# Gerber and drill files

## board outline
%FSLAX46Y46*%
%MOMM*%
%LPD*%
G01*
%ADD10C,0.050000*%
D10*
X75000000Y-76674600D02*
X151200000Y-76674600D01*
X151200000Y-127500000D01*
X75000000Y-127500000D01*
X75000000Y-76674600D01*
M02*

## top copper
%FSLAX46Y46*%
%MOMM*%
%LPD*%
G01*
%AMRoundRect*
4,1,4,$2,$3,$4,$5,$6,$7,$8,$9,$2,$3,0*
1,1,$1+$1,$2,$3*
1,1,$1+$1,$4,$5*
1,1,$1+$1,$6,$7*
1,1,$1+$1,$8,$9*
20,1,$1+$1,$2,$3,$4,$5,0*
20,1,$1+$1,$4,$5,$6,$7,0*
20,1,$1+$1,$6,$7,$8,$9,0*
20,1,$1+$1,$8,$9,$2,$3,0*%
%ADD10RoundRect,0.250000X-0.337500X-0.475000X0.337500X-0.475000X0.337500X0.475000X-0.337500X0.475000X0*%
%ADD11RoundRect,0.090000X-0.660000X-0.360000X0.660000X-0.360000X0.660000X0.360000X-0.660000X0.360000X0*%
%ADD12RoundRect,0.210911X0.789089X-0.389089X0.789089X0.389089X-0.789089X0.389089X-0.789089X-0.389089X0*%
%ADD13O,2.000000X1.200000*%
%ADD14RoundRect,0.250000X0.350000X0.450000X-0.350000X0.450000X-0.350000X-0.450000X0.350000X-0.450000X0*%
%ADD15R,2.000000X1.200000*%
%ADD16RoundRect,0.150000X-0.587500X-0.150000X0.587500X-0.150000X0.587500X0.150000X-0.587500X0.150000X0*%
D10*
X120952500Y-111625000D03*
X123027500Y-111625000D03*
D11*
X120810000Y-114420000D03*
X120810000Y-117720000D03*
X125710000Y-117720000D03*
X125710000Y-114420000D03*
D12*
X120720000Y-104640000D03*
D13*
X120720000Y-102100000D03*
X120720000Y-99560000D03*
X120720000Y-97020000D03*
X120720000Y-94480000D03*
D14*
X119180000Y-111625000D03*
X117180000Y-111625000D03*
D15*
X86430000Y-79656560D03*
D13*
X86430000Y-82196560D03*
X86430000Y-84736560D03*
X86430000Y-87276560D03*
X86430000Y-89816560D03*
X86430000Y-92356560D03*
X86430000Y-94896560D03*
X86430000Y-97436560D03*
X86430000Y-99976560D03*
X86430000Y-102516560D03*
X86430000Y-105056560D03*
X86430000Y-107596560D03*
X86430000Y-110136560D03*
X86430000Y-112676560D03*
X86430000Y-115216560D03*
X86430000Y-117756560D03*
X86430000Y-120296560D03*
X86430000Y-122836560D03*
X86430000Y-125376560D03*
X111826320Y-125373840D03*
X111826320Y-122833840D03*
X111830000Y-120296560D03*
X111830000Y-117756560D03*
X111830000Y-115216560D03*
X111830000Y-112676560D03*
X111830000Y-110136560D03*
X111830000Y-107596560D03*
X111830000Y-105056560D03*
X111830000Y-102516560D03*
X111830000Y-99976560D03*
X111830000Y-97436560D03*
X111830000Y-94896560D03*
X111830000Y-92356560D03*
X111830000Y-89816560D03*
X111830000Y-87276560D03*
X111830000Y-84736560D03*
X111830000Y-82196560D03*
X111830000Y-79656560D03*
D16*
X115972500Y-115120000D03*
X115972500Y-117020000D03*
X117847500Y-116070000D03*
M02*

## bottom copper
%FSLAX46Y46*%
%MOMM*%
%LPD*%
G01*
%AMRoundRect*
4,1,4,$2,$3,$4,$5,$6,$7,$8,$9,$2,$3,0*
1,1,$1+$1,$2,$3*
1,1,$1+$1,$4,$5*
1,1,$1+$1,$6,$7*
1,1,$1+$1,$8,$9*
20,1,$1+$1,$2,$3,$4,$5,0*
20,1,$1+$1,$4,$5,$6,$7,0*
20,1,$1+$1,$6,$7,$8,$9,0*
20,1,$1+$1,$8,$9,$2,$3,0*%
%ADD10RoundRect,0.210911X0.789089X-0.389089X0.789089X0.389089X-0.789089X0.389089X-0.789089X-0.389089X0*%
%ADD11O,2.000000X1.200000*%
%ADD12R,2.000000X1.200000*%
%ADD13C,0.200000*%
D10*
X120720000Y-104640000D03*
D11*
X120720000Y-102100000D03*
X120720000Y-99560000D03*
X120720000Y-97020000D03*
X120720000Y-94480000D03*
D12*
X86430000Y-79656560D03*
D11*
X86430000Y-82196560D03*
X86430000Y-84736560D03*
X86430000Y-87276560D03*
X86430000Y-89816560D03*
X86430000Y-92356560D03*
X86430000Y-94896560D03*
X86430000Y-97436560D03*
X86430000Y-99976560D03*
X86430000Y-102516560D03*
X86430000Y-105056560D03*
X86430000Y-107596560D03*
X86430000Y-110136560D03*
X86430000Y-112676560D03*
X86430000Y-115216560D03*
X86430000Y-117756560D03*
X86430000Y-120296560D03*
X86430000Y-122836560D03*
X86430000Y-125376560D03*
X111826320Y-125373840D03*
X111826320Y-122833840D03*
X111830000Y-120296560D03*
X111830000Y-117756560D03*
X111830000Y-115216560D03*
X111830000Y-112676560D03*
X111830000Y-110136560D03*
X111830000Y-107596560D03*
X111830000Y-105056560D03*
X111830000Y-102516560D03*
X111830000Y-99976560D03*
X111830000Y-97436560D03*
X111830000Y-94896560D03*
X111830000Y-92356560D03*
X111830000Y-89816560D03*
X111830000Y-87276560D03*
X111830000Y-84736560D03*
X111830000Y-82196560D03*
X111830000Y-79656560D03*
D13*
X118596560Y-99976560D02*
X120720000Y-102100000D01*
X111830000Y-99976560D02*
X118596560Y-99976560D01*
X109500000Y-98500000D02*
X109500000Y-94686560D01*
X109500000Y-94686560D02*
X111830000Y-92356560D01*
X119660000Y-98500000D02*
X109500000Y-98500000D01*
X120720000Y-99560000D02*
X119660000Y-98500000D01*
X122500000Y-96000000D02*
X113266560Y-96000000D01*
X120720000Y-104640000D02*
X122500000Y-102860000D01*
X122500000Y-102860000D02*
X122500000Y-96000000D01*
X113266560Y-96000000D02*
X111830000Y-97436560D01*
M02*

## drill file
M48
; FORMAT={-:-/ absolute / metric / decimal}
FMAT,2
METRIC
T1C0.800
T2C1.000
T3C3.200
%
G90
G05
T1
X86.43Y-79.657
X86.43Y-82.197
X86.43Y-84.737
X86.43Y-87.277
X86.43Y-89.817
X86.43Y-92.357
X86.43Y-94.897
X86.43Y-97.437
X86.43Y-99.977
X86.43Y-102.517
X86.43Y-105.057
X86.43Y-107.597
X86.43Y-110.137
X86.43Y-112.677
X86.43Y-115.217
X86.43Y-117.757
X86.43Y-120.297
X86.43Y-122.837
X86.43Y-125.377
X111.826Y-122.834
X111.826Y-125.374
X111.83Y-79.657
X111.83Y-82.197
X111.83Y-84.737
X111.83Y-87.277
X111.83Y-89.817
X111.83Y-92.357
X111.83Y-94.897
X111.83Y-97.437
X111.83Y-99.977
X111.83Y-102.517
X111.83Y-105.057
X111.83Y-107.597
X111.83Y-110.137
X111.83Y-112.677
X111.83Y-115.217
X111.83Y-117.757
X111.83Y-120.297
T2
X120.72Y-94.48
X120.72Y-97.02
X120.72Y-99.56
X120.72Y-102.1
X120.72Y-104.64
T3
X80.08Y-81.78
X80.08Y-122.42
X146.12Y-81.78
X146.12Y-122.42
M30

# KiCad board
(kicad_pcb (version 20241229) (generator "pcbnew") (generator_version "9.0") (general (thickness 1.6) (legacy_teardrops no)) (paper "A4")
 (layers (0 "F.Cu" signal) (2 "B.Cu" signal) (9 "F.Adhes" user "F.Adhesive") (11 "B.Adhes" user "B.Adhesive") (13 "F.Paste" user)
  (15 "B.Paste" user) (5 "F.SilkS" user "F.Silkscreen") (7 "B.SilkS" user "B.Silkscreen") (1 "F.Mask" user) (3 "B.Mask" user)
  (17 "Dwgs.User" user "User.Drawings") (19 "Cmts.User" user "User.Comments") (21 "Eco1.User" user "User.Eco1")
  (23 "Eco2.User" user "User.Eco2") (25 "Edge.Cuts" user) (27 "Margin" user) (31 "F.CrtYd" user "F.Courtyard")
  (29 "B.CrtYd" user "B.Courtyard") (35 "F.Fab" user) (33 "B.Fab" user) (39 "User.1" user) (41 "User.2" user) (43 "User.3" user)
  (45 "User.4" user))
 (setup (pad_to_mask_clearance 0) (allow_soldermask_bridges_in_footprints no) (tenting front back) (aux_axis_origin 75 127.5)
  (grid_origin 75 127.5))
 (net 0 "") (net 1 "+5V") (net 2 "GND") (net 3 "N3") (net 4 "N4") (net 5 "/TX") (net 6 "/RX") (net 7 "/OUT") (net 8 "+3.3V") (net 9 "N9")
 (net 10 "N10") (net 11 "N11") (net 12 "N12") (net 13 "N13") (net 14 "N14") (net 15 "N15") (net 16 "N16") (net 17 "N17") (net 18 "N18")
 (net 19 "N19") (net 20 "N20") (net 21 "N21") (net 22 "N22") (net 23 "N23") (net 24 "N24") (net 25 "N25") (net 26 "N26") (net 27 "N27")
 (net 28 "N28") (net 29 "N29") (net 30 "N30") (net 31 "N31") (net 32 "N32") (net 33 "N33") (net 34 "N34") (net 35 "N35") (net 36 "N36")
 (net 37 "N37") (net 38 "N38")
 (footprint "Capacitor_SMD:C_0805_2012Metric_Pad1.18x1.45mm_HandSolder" (layer "F.Cu") (at 121.99 111.625)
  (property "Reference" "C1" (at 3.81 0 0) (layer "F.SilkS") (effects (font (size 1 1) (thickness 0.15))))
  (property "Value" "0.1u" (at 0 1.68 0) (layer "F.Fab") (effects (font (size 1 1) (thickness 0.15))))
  (pad "1" smd roundrect (at -1.0375 0) (size 1.175 1.45) (layers "F.Cu" "F.Mask" "F.Paste") (roundrect_rratio 0.212766) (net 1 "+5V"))
  (pad "2" smd roundrect (at 1.0375 0) (size 1.175 1.45) (layers "F.Cu" "F.Mask" "F.Paste") (roundrect_rratio 0.212766) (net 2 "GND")))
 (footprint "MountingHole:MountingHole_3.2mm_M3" (layer "F.Cu") (at 146.12 81.78)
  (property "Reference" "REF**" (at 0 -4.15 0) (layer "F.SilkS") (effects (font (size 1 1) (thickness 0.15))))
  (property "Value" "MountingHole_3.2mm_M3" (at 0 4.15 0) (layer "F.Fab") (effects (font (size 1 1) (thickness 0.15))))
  (pad "" np_thru_hole circle (at 0 0) (size 3.2 3.2) (drill 3.2) (layers "*.Cu" "*.Mask")))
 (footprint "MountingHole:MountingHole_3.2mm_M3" (layer "F.Cu") (at 80.08 122.42)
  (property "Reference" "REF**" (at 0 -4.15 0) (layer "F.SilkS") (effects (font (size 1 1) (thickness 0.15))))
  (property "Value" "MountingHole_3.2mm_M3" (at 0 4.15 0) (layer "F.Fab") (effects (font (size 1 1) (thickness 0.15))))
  (pad "" np_thru_hole circle (at 0 0) (size 3.2 3.2) (drill 3.2) (layers "*.Cu" "*.Mask")))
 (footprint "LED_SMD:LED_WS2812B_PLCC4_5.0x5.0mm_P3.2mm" (layer "F.Cu") (at 123.26 116.07)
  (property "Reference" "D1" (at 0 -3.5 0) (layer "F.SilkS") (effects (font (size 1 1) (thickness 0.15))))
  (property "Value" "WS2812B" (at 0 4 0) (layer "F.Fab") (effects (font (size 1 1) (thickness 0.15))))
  (pad "1" smd roundrect (at -2.45 -1.65) (size 1.5 0.9) (layers "F.Cu" "F.Mask" "F.Paste") (roundrect_rratio 0.1) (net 1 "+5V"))
  (pad "2" smd roundrect (at -2.45 1.65) (size 1.5 0.9) (layers "F.Cu" "F.Mask" "F.Paste") (roundrect_rratio 0.1) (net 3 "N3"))
  (pad "3" smd roundrect (at 2.45 1.65) (size 1.5 0.9) (layers "F.Cu" "F.Mask" "F.Paste") (roundrect_rratio 0.1) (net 2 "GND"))
  (pad "4" smd roundrect (at 2.45 -1.65) (size 1.5 0.9) (layers "F.Cu" "F.Mask" "F.Paste") (roundrect_rratio 0.1) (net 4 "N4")))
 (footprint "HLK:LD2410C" (layer "F.Cu") (at 120.72 104.64 90)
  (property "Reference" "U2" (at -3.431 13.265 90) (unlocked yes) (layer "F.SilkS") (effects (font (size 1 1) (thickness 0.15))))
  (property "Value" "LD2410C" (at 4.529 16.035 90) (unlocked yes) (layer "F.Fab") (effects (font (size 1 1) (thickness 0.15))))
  (pad "1" thru_hole roundrect (at 0 0 90) (size 1.2 2) (drill 1) (layers "*.Cu" "*.Mask") (remove_unused_layers no)
   (roundrect_rratio 0.1757592801) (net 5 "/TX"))
  (pad "2" thru_hole oval (at 2.54 0 90) (size 1.2 2) (drill 1) (layers "*.Cu" "*.Mask") (remove_unused_layers no) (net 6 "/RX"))
  (pad "3" thru_hole oval (at 5.08 0 90) (size 1.2 2) (drill 1) (layers "*.Cu" "*.Mask") (remove_unused_layers no) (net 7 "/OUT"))
  (pad "4" thru_hole oval (at 7.62 0 90) (size 1.2 2) (drill 1) (layers "*.Cu" "*.Mask") (remove_unused_layers no) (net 2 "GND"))
  (pad "5" thru_hole oval (at 10.16 0 90) (size 1.2 2) (drill 1) (layers "*.Cu" "*.Mask") (remove_unused_layers no) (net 1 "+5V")))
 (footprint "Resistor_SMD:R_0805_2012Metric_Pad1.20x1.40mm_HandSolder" (layer "F.Cu") (at 118.18 111.625 180)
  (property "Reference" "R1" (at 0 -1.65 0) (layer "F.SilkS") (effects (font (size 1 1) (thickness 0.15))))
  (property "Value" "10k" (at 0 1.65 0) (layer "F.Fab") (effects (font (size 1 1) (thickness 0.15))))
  (pad "1" smd roundrect (at -1 0 180) (size 1.2 1.4) (layers "F.Cu" "F.Mask" "F.Paste") (roundrect_rratio 0.208333) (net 1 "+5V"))
  (pad "2" smd roundrect (at 1 0 180) (size 1.2 1.4) (layers "F.Cu" "F.Mask" "F.Paste") (roundrect_rratio 0.208333) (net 4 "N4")))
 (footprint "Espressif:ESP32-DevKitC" (layer "F.Cu") (at 86.43 79.65656)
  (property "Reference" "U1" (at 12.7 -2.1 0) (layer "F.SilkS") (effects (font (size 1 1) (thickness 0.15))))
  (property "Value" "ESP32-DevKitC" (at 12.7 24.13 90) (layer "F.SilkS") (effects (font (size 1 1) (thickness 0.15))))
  (pad "1" thru_hole rect (at 0 0 270) (size 1.2 2) (drill 0.8) (layers "*.Cu" "*.Mask") (remove_unused_layers no) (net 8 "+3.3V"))
  (pad "2" thru_hole oval (at 0 2.54 270) (size 1.2 2) (drill 0.8) (layers "*.Cu" "*.Mask") (remove_unused_layers no) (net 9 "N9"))
  (pad "3" thru_hole oval (at 0 5.08 270) (size 1.2 2) (drill 0.8) (layers "*.Cu" "*.Mask") (remove_unused_layers no) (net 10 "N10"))
  (pad "4" thru_hole oval (at 0 7.62 270) (size 1.2 2) (drill 0.8) (layers "*.Cu" "*.Mask") (remove_unused_layers no) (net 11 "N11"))
  (pad "5" thru_hole oval (at 0 10.16 270) (size 1.2 2) (drill 0.8) (layers "*.Cu" "*.Mask") (remove_unused_layers no) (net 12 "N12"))
  (pad "6" thru_hole oval (at 0 12.7 270) (size 1.2 2) (drill 0.8) (layers "*.Cu" "*.Mask") (remove_unused_layers no) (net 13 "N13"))
  (pad "7" thru_hole oval (at 0 15.24 270) (size 1.2 2) (drill 0.8) (layers "*.Cu" "*.Mask") (remove_unused_layers no) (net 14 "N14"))
  (pad "8" thru_hole oval (at 0 17.78 270) (size 1.2 2) (drill 0.8) (layers "*.Cu" "*.Mask") (remove_unused_layers no) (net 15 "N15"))
  (pad "9" thru_hole oval (at 0 20.32 270) (size 1.2 2) (drill 0.8) (layers "*.Cu" "*.Mask") (remove_unused_layers no) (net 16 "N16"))
  (pad "10" thru_hole oval (at 0 22.86 270) (size 1.2 2) (drill 0.8) (layers "*.Cu" "*.Mask") (remove_unused_layers no) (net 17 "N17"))
  (pad "11" thru_hole oval (at 0 25.4 270) (size 1.2 2) (drill 0.8) (layers "*.Cu" "*.Mask") (remove_unused_layers no) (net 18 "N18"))
  (pad "12" thru_hole oval (at 0 27.94 270) (size 1.2 2) (drill 0.8) (layers "*.Cu" "*.Mask") (remove_unused_layers no) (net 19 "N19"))
  (pad "13" thru_hole oval (at 0 30.48 270) (size 1.2 2) (drill 0.8) (layers "*.Cu" "*.Mask") (remove_unused_layers no) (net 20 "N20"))
  (pad "14" thru_hole oval (at 0 33.02 270) (size 1.2 2) (drill 0.8) (layers "*.Cu" "*.Mask") (remove_unused_layers no) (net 2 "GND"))
  (pad "15" thru_hole oval (at 0 35.56 270) (size 1.2 2) (drill 0.8) (layers "*.Cu" "*.Mask") (remove_unused_layers no) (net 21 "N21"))
  (pad "16" thru_hole oval (at 0 38.1 270) (size 1.2 2) (drill 0.8) (layers "*.Cu" "*.Mask") (remove_unused_layers no) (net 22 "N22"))
  (pad "17" thru_hole oval (at 0 40.64 270) (size 1.2 2) (drill 0.8) (layers "*.Cu" "*.Mask") (remove_unused_layers no) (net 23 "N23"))
  (pad "18" thru_hole oval (at 0 43.18 270) (size 1.2 2) (drill 0.8) (layers "*.Cu" "*.Mask") (remove_unused_layers no) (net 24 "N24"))
  (pad "19" thru_hole oval (at 0 45.72 270) (size 1.2 2) (drill 0.8) (layers "*.Cu" "*.Mask") (remove_unused_layers no) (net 1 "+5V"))
  (pad "20" thru_hole oval (at 25.39632 45.71728 270) (size 1.2 2) (drill 0.8) (layers "*.Cu" "*.Mask") (remove_unused_layers no)
   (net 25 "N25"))
  (pad "21" thru_hole oval (at 25.39632 43.17728 270) (size 1.2 2) (drill 0.8) (layers "*.Cu" "*.Mask") (remove_unused_layers no)
   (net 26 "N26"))
  (pad "22" thru_hole oval (at 25.4 40.64 270) (size 1.2 2) (drill 0.8) (layers "*.Cu" "*.Mask") (remove_unused_layers no) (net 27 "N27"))
  (pad "23" thru_hole oval (at 25.4 38.1 270) (size 1.2 2) (drill 0.8) (layers "*.Cu" "*.Mask") (remove_unused_layers no) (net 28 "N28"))
  (pad "24" thru_hole oval (at 25.4 35.56 270) (size 1.2 2) (drill 0.8) (layers "*.Cu" "*.Mask") (remove_unused_layers no) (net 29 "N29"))
  (pad "25" thru_hole oval (at 25.4 33.02 270) (size 1.2 2) (drill 0.8) (layers "*.Cu" "*.Mask") (remove_unused_layers no) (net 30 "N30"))
  (pad "26" thru_hole oval (at 25.4 30.48 270) (size 1.2 2) (drill 0.8) (layers "*.Cu" "*.Mask") (remove_unused_layers no) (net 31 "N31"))
  (pad "27" thru_hole oval (at 25.4 27.94 270) (size 1.2 2) (drill 0.8) (layers "*.Cu" "*.Mask") (remove_unused_layers no) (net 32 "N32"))
  (pad "28" thru_hole oval (at 25.4 25.4 270) (size 1.2 2) (drill 0.8) (layers "*.Cu" "*.Mask") (remove_unused_layers no) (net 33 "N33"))
  (pad "29" thru_hole oval (at 25.4 22.86 270) (size 1.2 2) (drill 0.8) (layers "*.Cu" "*.Mask") (remove_unused_layers no) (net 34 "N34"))
  (pad "30" thru_hole oval (at 25.4 20.32 270) (size 1.2 2) (drill 0.8) (layers "*.Cu" "*.Mask") (remove_unused_layers no) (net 6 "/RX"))
  (pad "31" thru_hole oval (at 25.4 17.78 270) (size 1.2 2) (drill 0.8) (layers "*.Cu" "*.Mask") (remove_unused_layers no) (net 5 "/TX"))
  (pad "32" thru_hole oval (at 25.4 15.24 270) (size 1.2 2) (drill 0.8) (layers "*.Cu" "*.Mask") (remove_unused_layers no) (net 2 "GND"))
  (pad "33" thru_hole oval (at 25.4 12.7 270) (size 1.2 2) (drill 0.8) (layers "*.Cu" "*.Mask") (remove_unused_layers no) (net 7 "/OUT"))
  (pad "34" thru_hole oval (at 25.4 10.16 270) (size 1.2 2) (drill 0.8) (layers "*.Cu" "*.Mask") (remove_unused_layers no) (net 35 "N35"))
  (pad "35" thru_hole oval (at 25.4 7.62 270) (size 1.2 2) (drill 0.8) (layers "*.Cu" "*.Mask") (remove_unused_layers no) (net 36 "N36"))
  (pad "36" thru_hole oval (at 25.4 5.08 270) (size 1.2 2) (drill 0.8) (layers "*.Cu" "*.Mask") (remove_unused_layers no) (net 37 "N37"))
  (pad "37" thru_hole oval (at 25.4 2.54 270) (size 1.2 2) (drill 0.8) (layers "*.Cu" "*.Mask") (remove_unused_layers no) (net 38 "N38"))
  (pad "38" thru_hole oval (at 25.4 0 270) (size 1.2 2) (drill 0.8) (layers "*.Cu" "*.Mask") (remove_unused_layers no) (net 2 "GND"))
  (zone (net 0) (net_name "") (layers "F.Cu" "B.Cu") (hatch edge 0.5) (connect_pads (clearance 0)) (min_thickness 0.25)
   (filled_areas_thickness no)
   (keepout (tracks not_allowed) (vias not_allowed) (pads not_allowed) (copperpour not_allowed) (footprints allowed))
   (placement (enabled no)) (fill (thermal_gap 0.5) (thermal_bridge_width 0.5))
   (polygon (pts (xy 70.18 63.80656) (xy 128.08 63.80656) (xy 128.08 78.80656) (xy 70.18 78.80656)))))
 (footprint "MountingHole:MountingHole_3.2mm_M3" (layer "F.Cu") (at 146.12 122.42)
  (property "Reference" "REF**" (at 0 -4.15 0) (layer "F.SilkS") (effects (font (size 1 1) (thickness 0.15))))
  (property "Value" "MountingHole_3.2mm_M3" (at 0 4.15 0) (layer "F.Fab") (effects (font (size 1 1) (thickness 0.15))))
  (pad "" np_thru_hole circle (at 0 0) (size 3.2 3.2) (drill 3.2) (layers "*.Cu" "*.Mask")))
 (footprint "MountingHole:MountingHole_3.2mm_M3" (layer "F.Cu") (at 80.08 81.78)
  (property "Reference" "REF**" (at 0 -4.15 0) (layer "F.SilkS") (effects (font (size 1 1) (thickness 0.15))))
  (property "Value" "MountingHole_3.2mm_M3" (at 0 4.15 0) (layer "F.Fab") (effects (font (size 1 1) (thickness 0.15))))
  (pad "" np_thru_hole circle (at 0 0) (size 3.2 3.2) (drill 3.2) (layers "*.Cu" "*.Mask")))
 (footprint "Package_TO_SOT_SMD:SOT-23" (layer "F.Cu") (at 116.91 116.07)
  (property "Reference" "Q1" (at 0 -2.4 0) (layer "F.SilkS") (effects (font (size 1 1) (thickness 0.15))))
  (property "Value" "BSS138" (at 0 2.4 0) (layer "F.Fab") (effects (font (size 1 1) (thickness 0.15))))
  (pad "1" smd roundrect (at -0.9375 -0.95) (size 1.475 0.6) (layers "F.Cu" "F.Mask" "F.Paste") (roundrect_rratio 0.25) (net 8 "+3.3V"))
  (pad "2" smd roundrect (at -0.9375 0.95) (size 1.475 0.6) (layers "F.Cu" "F.Mask" "F.Paste") (roundrect_rratio 0.25) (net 37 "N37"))
  (pad "3" smd roundrect (at 0.9375 0) (size 1.475 0.6) (layers "F.Cu" "F.Mask" "F.Paste") (roundrect_rratio 0.25) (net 4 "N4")))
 (gr_rect (start 75 76.6746) (end 151.2 127.5) (stroke (width 0.05) (type default)) (fill no) (layer "Edge.Cuts"))
 (segment (start 118.59656 99.97656) (end 120.72 102.1) (width 0.2) (layer "B.Cu") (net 6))
 (segment (start 111.83 99.97656) (end 118.59656 99.97656) (width 0.2) (layer "B.Cu") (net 6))
 (segment (start 109.5 98.5) (end 109.5 94.68656) (width 0.2) (layer "B.Cu") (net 7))
 (segment (start 109.5 94.68656) (end 111.83 92.35656) (width 0.2) (layer "B.Cu") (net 7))
 (segment (start 119.66 98.5) (end 109.5 98.5) (width 0.2) (layer "B.Cu") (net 7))
 (segment (start 120.72 99.56) (end 119.66 98.5) (width 0.2) (layer "B.Cu") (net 7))
 (segment (start 122.5 96) (end 113.26656 96) (width 0.2) (layer "B.Cu") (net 5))
 (segment (start 120.72 104.64) (end 122.5 102.86) (width 0.2) (layer "B.Cu") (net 5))
 (segment (start 122.5 102.86) (end 122.5 96) (width 0.2) (layer "B.Cu") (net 5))
 (segment (start 113.26656 96) (end 111.83 97.43656) (width 0.2) (layer "B.Cu") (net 5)))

